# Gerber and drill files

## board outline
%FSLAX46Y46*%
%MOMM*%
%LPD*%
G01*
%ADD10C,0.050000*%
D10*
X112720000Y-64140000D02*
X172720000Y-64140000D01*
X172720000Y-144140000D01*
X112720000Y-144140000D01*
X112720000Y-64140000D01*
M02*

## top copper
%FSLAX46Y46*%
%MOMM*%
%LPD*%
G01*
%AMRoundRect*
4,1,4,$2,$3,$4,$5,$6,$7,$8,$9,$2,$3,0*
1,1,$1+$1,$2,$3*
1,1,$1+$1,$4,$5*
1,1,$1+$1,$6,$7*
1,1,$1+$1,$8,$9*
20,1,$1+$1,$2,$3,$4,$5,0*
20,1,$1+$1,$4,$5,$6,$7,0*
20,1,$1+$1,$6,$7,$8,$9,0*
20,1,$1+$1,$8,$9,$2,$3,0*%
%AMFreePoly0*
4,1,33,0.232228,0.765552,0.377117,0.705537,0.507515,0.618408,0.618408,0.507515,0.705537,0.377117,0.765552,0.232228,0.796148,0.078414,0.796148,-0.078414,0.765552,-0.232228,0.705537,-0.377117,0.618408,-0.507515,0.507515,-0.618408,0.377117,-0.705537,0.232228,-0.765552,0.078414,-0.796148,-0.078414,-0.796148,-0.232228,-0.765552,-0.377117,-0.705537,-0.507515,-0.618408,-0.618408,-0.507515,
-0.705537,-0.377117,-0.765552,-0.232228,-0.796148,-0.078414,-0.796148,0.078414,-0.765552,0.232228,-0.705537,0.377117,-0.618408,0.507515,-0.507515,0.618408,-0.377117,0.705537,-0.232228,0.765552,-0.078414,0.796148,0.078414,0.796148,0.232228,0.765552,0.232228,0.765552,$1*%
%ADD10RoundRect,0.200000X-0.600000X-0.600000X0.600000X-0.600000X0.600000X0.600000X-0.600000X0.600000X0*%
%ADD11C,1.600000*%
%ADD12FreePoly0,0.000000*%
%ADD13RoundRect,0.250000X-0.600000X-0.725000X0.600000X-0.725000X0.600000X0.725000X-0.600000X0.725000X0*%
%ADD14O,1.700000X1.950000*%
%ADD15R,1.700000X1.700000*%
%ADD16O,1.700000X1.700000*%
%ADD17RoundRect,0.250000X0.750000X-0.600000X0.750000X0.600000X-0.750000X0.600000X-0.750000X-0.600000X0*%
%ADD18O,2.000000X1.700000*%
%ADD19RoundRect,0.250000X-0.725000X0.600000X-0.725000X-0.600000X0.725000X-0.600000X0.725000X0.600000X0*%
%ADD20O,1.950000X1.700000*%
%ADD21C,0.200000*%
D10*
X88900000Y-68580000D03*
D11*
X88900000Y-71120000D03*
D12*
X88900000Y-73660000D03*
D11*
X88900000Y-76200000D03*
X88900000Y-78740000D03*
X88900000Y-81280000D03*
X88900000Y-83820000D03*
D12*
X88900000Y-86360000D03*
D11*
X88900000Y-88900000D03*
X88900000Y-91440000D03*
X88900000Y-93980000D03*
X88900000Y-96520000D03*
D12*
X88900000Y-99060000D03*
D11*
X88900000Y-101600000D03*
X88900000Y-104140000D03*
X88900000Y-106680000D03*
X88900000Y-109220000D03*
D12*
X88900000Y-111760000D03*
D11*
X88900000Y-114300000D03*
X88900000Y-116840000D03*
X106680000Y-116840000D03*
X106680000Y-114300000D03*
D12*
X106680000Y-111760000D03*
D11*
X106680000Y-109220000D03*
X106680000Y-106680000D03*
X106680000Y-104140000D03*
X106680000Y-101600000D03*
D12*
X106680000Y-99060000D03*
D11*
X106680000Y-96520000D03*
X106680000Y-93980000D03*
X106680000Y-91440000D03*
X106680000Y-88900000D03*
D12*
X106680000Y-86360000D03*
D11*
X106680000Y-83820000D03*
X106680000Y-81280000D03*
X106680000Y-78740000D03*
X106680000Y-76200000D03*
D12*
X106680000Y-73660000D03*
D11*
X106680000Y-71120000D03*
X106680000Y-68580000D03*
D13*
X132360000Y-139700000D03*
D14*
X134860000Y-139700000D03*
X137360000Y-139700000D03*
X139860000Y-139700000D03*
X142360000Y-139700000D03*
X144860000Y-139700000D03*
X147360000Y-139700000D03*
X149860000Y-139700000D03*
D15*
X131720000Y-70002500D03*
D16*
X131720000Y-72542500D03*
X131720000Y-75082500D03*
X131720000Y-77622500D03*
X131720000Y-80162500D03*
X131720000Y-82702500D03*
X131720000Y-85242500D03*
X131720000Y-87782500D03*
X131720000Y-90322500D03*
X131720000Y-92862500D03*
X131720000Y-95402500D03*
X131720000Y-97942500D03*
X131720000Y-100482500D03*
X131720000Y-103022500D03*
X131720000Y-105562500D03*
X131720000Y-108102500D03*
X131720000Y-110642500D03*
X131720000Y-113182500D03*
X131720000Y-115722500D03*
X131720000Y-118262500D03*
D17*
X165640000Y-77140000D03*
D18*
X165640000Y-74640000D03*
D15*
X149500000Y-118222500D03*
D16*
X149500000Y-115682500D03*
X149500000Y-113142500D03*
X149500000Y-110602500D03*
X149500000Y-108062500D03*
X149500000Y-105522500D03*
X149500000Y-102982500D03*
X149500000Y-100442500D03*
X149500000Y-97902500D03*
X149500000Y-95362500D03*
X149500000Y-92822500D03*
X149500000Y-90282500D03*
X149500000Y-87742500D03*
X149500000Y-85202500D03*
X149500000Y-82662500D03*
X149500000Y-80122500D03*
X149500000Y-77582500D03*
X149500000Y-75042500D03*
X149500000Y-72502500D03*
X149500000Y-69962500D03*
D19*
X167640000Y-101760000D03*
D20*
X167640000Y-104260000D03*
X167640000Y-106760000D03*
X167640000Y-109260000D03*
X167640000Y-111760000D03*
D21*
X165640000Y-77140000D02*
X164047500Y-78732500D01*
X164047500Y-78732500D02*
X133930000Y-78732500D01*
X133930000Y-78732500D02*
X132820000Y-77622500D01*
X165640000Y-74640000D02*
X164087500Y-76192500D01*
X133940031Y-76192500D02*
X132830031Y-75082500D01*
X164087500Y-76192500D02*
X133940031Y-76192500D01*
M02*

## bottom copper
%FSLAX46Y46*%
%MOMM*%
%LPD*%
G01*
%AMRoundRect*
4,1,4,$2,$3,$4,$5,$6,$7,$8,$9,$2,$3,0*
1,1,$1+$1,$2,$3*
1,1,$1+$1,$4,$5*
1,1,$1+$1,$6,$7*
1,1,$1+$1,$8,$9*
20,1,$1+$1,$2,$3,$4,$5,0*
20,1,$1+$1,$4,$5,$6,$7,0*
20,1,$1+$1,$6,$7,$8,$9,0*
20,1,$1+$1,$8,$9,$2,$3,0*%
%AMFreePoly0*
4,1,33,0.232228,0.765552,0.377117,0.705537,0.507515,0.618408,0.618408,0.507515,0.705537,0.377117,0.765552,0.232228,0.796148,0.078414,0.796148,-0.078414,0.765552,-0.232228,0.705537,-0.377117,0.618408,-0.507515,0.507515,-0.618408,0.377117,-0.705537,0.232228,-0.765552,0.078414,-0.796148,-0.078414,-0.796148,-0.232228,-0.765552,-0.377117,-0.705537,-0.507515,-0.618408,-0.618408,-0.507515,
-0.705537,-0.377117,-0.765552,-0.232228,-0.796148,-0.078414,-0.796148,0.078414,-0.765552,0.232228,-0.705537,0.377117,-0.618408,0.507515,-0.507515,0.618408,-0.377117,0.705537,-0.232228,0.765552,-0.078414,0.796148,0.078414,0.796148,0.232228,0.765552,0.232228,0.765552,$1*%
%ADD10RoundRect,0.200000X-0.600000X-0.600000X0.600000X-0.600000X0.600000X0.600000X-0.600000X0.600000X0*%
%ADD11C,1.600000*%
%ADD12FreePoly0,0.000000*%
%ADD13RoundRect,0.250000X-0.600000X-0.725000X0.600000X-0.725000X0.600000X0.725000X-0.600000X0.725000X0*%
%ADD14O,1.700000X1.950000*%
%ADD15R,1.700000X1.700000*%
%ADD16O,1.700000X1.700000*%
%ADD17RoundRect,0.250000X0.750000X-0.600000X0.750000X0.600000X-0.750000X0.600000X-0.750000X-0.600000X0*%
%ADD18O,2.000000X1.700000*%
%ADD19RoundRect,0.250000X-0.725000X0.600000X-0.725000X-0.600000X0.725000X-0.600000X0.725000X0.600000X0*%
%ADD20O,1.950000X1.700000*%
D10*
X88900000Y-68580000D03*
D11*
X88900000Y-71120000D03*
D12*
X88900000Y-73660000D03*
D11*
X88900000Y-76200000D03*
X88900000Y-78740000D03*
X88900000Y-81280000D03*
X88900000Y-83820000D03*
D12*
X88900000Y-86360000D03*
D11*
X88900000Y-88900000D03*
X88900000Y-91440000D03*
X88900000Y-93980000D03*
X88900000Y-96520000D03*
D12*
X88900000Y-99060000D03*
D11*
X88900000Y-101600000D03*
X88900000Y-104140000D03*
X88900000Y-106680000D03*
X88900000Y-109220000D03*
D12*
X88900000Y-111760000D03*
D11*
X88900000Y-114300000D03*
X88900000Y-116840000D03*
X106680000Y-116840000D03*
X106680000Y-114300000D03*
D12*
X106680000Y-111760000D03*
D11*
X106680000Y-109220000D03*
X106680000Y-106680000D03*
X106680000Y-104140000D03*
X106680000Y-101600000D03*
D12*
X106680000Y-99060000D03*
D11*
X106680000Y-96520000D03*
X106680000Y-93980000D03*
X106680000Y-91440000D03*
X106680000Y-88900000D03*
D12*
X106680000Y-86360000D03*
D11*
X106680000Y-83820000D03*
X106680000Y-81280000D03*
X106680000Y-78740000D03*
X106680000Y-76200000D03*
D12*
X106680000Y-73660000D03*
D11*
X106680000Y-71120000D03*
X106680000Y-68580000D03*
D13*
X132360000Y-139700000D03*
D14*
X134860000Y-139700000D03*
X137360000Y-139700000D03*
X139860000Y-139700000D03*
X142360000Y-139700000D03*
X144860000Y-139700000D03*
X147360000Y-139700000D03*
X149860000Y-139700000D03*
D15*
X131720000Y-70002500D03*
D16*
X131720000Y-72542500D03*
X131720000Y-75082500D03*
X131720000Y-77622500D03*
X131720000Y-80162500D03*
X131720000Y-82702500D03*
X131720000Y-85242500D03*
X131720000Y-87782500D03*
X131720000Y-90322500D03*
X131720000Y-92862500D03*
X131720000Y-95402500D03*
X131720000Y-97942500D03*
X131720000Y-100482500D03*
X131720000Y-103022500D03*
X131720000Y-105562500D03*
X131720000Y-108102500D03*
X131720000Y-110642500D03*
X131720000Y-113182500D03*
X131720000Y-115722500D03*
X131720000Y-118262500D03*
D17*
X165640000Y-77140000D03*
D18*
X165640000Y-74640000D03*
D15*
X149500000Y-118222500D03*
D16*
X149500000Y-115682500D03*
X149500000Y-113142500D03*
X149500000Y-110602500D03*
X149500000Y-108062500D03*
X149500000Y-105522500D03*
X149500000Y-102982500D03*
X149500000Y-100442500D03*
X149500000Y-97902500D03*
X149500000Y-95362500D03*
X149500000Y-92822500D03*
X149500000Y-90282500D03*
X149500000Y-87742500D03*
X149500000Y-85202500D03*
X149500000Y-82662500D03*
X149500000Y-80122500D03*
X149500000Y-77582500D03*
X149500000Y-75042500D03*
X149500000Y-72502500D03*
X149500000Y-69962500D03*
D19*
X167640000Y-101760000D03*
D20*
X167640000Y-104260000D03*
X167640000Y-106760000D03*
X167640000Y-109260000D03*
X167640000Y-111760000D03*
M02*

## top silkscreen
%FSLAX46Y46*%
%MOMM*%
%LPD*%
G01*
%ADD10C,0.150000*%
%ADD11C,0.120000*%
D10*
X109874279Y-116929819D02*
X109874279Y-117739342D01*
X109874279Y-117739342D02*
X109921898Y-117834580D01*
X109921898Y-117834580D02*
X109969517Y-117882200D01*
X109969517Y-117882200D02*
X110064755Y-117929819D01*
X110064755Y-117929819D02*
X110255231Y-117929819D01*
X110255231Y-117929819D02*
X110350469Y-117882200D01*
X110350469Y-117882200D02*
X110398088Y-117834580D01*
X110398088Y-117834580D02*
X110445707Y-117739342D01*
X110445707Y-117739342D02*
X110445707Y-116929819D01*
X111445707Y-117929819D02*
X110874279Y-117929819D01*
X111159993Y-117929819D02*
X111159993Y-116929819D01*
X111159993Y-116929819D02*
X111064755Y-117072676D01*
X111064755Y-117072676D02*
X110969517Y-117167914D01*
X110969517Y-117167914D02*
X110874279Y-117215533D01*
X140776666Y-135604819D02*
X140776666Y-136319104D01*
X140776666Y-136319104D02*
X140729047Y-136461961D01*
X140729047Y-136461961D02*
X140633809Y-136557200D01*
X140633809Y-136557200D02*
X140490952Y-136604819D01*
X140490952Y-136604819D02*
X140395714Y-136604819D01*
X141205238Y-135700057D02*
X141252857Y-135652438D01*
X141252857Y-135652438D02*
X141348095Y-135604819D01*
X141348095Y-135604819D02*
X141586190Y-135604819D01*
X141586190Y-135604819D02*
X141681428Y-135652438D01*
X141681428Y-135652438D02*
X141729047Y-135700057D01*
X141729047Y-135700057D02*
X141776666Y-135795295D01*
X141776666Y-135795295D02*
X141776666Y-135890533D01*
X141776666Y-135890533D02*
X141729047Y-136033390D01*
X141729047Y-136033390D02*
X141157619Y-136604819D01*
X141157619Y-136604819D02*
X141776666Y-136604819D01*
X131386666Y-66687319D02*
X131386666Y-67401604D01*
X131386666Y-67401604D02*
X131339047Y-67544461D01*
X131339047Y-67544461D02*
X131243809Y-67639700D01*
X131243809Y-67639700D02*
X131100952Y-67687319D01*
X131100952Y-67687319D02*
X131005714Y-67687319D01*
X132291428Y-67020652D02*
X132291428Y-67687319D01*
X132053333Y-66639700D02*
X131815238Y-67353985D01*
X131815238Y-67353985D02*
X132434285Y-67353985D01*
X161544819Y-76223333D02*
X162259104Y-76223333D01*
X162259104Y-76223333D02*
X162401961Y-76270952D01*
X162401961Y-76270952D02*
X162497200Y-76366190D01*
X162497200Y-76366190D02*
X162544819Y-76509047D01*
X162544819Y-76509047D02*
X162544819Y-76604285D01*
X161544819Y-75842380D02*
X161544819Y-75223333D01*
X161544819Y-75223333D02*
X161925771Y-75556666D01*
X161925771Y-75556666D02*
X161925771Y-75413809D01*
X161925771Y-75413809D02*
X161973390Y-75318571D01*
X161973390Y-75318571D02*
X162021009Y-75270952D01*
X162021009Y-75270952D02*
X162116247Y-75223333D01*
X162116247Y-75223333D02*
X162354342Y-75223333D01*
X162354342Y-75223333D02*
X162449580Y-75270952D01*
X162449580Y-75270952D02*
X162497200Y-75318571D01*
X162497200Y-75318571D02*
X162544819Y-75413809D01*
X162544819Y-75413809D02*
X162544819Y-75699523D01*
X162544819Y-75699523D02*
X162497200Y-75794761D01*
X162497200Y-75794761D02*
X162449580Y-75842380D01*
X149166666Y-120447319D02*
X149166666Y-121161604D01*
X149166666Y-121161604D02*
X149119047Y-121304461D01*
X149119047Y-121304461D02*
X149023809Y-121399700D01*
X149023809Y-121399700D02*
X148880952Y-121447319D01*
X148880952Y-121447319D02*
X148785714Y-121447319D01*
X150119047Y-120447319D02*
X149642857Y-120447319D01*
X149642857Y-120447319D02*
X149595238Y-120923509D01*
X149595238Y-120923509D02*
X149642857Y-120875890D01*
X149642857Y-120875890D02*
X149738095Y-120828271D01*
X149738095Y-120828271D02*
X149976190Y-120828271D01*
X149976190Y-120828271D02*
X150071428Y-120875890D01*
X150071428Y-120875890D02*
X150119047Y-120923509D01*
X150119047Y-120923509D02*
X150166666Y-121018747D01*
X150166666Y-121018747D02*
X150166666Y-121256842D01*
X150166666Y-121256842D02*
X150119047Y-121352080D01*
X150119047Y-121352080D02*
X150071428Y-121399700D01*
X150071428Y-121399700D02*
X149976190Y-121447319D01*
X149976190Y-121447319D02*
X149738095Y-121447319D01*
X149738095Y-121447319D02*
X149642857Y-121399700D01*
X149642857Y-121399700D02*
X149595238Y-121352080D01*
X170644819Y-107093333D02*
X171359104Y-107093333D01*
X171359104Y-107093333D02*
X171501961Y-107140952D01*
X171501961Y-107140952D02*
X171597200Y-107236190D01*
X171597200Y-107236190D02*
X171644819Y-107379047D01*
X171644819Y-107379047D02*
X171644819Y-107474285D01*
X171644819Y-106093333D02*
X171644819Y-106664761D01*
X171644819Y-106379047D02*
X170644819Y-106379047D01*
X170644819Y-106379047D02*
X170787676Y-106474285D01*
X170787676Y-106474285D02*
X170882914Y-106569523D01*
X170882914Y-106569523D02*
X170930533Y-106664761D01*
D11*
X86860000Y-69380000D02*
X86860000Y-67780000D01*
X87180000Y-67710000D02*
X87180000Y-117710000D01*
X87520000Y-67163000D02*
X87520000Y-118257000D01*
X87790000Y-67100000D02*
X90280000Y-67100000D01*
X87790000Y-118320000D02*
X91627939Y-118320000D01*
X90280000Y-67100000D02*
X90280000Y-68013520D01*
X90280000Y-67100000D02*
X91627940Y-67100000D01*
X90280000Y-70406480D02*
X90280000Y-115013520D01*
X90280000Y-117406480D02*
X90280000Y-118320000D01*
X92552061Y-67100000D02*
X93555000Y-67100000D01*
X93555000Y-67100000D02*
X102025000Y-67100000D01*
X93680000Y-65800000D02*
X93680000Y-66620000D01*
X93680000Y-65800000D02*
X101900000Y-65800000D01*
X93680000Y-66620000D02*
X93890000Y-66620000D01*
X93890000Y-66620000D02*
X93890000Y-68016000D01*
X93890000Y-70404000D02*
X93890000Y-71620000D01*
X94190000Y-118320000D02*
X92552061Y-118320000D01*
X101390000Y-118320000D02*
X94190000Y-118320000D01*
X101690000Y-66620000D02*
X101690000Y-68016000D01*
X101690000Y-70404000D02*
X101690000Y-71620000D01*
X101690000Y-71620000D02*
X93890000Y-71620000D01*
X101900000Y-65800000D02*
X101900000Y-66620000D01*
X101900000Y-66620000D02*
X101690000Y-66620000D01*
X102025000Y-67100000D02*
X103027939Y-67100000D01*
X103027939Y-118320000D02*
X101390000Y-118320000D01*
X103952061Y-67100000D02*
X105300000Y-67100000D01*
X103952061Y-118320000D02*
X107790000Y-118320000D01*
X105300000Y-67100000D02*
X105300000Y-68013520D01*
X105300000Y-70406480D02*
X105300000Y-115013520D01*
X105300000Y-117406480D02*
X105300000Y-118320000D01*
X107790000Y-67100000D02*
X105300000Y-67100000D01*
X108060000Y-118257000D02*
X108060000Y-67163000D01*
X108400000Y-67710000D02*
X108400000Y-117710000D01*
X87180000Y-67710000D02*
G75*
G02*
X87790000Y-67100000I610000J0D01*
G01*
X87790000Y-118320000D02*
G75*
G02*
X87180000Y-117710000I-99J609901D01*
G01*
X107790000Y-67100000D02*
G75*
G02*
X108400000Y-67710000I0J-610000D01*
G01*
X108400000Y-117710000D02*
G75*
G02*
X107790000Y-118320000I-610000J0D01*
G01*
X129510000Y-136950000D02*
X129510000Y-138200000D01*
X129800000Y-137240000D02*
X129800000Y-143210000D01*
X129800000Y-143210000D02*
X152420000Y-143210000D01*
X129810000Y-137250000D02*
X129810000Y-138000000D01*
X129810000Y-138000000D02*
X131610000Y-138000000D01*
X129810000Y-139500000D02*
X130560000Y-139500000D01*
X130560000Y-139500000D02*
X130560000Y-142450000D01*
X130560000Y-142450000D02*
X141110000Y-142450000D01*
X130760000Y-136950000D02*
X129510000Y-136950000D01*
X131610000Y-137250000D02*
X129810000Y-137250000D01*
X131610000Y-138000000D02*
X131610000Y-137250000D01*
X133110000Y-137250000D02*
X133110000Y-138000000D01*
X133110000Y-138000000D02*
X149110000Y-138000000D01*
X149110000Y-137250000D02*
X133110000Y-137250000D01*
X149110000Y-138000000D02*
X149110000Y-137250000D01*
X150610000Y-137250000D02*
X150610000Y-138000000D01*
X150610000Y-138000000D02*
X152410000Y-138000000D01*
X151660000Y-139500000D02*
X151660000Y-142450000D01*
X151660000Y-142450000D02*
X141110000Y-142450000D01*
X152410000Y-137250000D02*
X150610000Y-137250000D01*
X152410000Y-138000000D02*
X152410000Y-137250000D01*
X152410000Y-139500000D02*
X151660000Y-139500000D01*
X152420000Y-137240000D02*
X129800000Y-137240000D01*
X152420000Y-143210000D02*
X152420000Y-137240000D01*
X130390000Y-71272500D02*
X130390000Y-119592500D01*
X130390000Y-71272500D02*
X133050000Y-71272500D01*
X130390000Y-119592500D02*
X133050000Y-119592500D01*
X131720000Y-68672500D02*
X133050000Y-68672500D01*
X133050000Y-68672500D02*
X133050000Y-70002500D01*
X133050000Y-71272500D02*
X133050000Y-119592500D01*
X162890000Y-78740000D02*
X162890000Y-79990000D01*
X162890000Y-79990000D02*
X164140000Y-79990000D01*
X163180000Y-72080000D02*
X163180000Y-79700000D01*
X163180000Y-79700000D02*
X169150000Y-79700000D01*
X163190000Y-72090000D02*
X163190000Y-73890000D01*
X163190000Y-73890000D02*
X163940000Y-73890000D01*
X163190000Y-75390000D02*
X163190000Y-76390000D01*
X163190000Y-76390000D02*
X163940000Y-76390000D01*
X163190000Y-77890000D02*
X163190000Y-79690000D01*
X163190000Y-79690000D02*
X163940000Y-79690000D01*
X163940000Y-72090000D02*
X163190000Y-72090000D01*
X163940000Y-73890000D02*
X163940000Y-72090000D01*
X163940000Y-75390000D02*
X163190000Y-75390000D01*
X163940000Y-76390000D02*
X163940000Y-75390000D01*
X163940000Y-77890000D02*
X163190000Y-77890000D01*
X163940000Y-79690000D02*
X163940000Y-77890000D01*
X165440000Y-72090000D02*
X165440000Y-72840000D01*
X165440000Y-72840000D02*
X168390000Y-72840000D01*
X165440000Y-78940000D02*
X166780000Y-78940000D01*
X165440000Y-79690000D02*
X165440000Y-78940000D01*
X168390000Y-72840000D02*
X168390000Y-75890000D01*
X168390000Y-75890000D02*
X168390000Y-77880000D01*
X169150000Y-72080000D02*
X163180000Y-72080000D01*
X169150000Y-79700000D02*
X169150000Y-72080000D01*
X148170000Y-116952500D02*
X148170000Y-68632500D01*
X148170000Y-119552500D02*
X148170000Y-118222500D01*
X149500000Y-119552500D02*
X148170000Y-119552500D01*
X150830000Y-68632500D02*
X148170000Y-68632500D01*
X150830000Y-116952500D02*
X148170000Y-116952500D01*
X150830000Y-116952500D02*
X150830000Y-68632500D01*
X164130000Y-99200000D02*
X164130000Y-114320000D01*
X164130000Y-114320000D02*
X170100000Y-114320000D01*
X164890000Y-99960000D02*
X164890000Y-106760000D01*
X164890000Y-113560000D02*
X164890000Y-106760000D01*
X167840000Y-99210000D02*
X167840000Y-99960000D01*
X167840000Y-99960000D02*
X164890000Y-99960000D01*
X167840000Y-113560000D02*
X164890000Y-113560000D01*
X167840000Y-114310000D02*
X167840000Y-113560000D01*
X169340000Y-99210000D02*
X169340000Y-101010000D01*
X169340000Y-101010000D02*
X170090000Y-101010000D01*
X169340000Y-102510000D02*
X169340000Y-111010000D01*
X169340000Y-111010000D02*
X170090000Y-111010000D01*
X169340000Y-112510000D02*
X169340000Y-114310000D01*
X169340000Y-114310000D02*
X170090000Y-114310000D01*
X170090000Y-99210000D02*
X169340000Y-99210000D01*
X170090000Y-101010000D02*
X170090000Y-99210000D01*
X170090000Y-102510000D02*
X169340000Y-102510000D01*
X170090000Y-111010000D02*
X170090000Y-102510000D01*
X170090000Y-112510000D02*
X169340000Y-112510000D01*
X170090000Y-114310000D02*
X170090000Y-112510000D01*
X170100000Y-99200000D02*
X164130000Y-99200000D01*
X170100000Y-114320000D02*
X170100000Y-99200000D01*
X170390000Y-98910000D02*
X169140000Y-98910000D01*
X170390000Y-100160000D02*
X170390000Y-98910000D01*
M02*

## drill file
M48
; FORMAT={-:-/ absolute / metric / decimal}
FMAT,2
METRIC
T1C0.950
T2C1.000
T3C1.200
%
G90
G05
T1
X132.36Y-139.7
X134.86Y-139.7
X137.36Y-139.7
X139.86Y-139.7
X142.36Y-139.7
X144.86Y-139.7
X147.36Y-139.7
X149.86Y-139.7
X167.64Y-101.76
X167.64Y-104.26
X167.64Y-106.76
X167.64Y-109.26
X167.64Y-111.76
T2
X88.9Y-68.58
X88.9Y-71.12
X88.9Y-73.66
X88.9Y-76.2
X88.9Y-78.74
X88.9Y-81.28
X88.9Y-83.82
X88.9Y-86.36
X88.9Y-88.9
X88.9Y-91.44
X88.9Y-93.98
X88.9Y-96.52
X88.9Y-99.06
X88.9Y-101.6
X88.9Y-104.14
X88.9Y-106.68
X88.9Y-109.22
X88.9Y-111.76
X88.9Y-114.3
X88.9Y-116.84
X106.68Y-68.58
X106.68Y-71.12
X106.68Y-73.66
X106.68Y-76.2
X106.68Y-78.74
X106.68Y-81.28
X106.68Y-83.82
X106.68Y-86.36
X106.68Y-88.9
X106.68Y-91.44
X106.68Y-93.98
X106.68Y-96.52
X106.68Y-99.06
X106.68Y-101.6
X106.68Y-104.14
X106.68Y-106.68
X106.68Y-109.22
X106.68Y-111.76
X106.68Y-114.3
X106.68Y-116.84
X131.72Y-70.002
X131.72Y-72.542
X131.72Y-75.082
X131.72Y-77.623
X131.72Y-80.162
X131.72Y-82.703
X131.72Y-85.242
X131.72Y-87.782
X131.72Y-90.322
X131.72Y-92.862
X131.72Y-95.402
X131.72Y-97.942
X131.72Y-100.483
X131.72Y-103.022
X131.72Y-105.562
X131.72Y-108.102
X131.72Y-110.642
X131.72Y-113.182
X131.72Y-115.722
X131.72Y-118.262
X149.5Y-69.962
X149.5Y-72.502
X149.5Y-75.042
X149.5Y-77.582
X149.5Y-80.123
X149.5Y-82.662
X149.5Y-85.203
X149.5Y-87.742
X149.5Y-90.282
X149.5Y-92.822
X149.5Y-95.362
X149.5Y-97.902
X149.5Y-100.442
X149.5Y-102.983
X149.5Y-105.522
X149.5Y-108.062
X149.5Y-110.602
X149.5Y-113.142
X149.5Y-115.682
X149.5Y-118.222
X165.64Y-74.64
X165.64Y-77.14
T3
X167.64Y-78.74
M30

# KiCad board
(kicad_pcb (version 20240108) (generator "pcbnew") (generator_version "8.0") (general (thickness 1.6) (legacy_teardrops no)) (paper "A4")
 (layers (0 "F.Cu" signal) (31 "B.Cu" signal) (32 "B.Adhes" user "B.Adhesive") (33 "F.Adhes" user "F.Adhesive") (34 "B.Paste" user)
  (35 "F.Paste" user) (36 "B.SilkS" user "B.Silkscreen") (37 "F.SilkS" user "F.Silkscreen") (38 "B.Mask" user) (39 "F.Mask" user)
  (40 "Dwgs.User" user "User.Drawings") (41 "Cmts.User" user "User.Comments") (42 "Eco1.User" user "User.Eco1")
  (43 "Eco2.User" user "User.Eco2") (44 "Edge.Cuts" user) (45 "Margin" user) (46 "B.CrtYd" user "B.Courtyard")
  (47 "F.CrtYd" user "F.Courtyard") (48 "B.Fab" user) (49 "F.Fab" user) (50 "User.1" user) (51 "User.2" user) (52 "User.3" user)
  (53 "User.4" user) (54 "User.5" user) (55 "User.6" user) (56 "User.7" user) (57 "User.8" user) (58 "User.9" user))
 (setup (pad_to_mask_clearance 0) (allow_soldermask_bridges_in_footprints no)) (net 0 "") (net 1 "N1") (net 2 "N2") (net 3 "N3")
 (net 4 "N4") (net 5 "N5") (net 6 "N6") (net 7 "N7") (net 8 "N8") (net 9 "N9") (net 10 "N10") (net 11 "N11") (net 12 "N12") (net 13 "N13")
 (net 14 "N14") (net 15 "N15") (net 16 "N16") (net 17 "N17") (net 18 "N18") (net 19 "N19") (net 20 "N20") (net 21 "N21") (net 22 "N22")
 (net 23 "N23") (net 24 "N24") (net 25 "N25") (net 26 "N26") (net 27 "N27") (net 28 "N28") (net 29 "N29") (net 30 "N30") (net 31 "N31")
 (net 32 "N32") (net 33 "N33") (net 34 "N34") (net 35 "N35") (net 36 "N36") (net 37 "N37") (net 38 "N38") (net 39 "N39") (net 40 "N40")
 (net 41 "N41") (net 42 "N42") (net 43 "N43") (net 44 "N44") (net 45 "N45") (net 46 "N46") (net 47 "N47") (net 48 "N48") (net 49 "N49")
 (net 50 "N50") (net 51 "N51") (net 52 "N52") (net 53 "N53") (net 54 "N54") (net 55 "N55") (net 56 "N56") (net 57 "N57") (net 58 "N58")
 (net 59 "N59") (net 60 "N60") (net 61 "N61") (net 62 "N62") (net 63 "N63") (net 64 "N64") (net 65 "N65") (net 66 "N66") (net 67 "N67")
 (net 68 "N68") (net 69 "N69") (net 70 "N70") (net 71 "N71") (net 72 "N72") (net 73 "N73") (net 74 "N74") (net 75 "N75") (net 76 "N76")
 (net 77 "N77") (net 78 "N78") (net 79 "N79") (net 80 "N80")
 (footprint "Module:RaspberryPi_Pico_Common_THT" (layer "F.Cu") (at 88.9 68.58)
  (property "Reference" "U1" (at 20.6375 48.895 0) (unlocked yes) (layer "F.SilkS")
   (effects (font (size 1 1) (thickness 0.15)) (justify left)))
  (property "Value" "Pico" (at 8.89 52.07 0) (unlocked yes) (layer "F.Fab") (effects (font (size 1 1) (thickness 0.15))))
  (fp_line (start -2.04 0.8) (end -2.04 -0.8) (stroke (width 0.12) (type solid)) (layer "F.SilkS"))
  (fp_line (start -1.72 -0.87) (end -1.72 49.13) (stroke (width 0.12) (type solid)) (layer "F.SilkS"))
  (fp_line (start -1.38 -1.417) (end -1.38 49.677) (stroke (width 0.12) (type solid)) (layer "F.SilkS"))
  (fp_line (start -1.11 -1.48) (end 1.38 -1.48) (stroke (width 0.12) (type solid)) (layer "F.SilkS"))
  (fp_line (start -1.11 49.74) (end 2.727939 49.74) (stroke (width 0.12) (type solid)) (layer "F.SilkS"))
  (fp_line (start 1.38 -1.48) (end 1.38 -0.56648) (stroke (width 0.12) (type solid)) (layer "F.SilkS"))
  (fp_line (start 1.38 -1.48) (end 2.72794 -1.48) (stroke (width 0.12) (type solid)) (layer "F.SilkS"))
  (fp_line (start 1.38 1.82648) (end 1.38 46.43352) (stroke (width 0.12) (type solid)) (layer "F.SilkS"))
  (fp_line (start 1.38 48.82648) (end 1.38 49.74) (stroke (width 0.12) (type solid)) (layer "F.SilkS"))
  (fp_line (start 3.652061 -1.48) (end 4.655 -1.48) (stroke (width 0.12) (type solid)) (layer "F.SilkS"))
  (fp_line (start 4.655 -1.48) (end 13.125 -1.48) (stroke (width 0.12) (type solid)) (layer "F.SilkS"))
  (fp_line (start 4.78 -2.78) (end 4.78 -1.96) (stroke (width 0.12) (type solid)) (layer "F.SilkS"))
  (fp_line (start 4.78 -2.78) (end 13 -2.78) (stroke (width 0.12) (type solid)) (layer "F.SilkS"))
  (fp_line (start 4.78 -1.96) (end 4.99 -1.96) (stroke (width 0.12) (type solid)) (layer "F.SilkS"))
  (fp_line (start 4.99 -1.96) (end 4.99 -0.564) (stroke (width 0.12) (type solid)) (layer "F.SilkS"))
  (fp_line (start 4.99 1.824) (end 4.99 3.04) (stroke (width 0.12) (type solid)) (layer "F.SilkS"))
  (fp_line (start 5.29 49.74) (end 3.652061 49.74) (stroke (width 0.12) (type solid)) (layer "F.SilkS"))
  (fp_line (start 12.49 49.74) (end 5.29 49.74) (stroke (width 0.12) (type solid)) (layer "F.SilkS"))
  (fp_line (start 12.79 -1.96) (end 12.79 -0.564) (stroke (width 0.12) (type solid)) (layer "F.SilkS"))
  (fp_line (start 12.79 1.824) (end 12.79 3.04) (stroke (width 0.12) (type solid)) (layer "F.SilkS"))
  (fp_line (start 12.79 3.04) (end 4.99 3.04) (stroke (width 0.12) (type solid)) (layer "F.SilkS"))
  (fp_line (start 13 -2.78) (end 13 -1.96) (stroke (width 0.12) (type solid)) (layer "F.SilkS"))
  (fp_line (start 13 -1.96) (end 12.79 -1.96) (stroke (width 0.12) (type solid)) (layer "F.SilkS"))
  (fp_line (start 13.125 -1.48) (end 14.127939 -1.48) (stroke (width 0.12) (type solid)) (layer "F.SilkS"))
  (fp_line (start 14.127939 49.74) (end 12.49 49.74) (stroke (width 0.12) (type solid)) (layer "F.SilkS"))
  (fp_line (start 15.052061 -1.48) (end 16.4 -1.48) (stroke (width 0.12) (type solid)) (layer "F.SilkS"))
  (fp_line (start 15.052061 49.74) (end 18.89 49.74) (stroke (width 0.12) (type solid)) (layer "F.SilkS"))
  (fp_line (start 16.4 -1.48) (end 16.4 -0.56648) (stroke (width 0.12) (type solid)) (layer "F.SilkS"))
  (fp_line (start 16.4 1.82648) (end 16.4 46.43352) (stroke (width 0.12) (type solid)) (layer "F.SilkS"))
  (fp_line (start 16.4 48.82648) (end 16.4 49.74) (stroke (width 0.12) (type solid)) (layer "F.SilkS"))
  (fp_line (start 18.89 -1.48) (end 16.4 -1.48) (stroke (width 0.12) (type solid)) (layer "F.SilkS"))
  (fp_line (start 19.16 49.677) (end 19.16 -1.417) (stroke (width 0.12) (type solid)) (layer "F.SilkS"))
  (fp_line (start 19.5 -0.87) (end 19.5 49.13) (stroke (width 0.12) (type solid)) (layer "F.SilkS"))
  (fp_arc (start -1.72 -0.87) (mid -1.541335 -1.301335) (end -1.11 -1.48) (stroke (width 0.12) (type solid)) (layer "F.SilkS"))
  (fp_arc (start -1.11 49.74) (mid -1.541364 49.561364) (end -1.72 49.13) (stroke (width 0.12) (type solid)) (layer "F.SilkS"))
  (fp_arc (start 18.89 -1.48) (mid 19.321335 -1.301335) (end 19.5 -0.87) (stroke (width 0.12) (type solid)) (layer "F.SilkS"))
  (fp_arc (start 19.5 49.13) (mid 19.321335 49.561335) (end 18.89 49.74) (stroke (width 0.12) (type solid)) (layer "F.SilkS"))
  (pad "1" thru_hole roundrect (at 0 0) (size 1.6 1.6) (drill 1) (layers "*.Cu" "*.Mask") (remove_unused_layers no) (roundrect_rratio 0.125)
   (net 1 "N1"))
  (pad "2" thru_hole circle (at 0 2.54) (size 1.6 1.6) (drill 1) (layers "*.Cu" "*.Mask") (remove_unused_layers no) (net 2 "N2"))
  (pad "3" thru_hole custom (at 0 5.08) (size 1.6 1.6) (drill 1) (layers "*.Cu" "*.Mask") (remove_unused_layers no) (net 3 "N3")
   (options (clearance outline) (anchor circle)) (primitives))
  (pad "4" thru_hole circle (at 0 7.62) (size 1.6 1.6) (drill 1) (layers "*.Cu" "*.Mask") (remove_unused_layers no) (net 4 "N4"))
  (pad "5" thru_hole circle (at 0 10.16) (size 1.6 1.6) (drill 1) (layers "*.Cu" "*.Mask") (remove_unused_layers no) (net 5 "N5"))
  (pad "6" thru_hole circle (at 0 12.7) (size 1.6 1.6) (drill 1) (layers "*.Cu" "*.Mask") (remove_unused_layers no) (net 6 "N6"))
  (pad "7" thru_hole circle (at 0 15.24) (size 1.6 1.6) (drill 1) (layers "*.Cu" "*.Mask") (remove_unused_layers no) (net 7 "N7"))
  (pad "8" thru_hole custom (at 0 17.78) (size 1.6 1.6) (drill 1) (layers "*.Cu" "*.Mask") (remove_unused_layers no) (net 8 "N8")
   (options (clearance outline) (anchor circle)) (primitives))
  (pad "9" thru_hole circle (at 0 20.32) (size 1.6 1.6) (drill 1) (layers "*.Cu" "*.Mask") (remove_unused_layers no) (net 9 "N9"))
  (pad "10" thru_hole circle (at 0 22.86) (size 1.6 1.6) (drill 1) (layers "*.Cu" "*.Mask") (remove_unused_layers no) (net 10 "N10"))
  (pad "11" thru_hole circle (at 0 25.4) (size 1.6 1.6) (drill 1) (layers "*.Cu" "*.Mask") (remove_unused_layers no) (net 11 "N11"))
  (pad "12" thru_hole circle (at 0 27.94) (size 1.6 1.6) (drill 1) (layers "*.Cu" "*.Mask") (remove_unused_layers no) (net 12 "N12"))
  (pad "13" thru_hole custom (at 0 30.48) (size 1.6 1.6) (drill 1) (layers "*.Cu" "*.Mask") (remove_unused_layers no) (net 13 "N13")
   (options (clearance outline) (anchor circle)) (primitives))
  (pad "14" thru_hole circle (at 0 33.02) (size 1.6 1.6) (drill 1) (layers "*.Cu" "*.Mask") (remove_unused_layers no) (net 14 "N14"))
  (pad "15" thru_hole circle (at 0 35.56) (size 1.6 1.6) (drill 1) (layers "*.Cu" "*.Mask") (remove_unused_layers no) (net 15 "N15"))
  (pad "16" thru_hole circle (at 0 38.1) (size 1.6 1.6) (drill 1) (layers "*.Cu" "*.Mask") (remove_unused_layers no) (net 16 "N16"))
  (pad "17" thru_hole circle (at 0 40.64) (size 1.6 1.6) (drill 1) (layers "*.Cu" "*.Mask") (remove_unused_layers no) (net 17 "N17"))
  (pad "18" thru_hole custom (at 0 43.18) (size 1.6 1.6) (drill 1) (layers "*.Cu" "*.Mask") (remove_unused_layers no) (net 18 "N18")
   (options (clearance outline) (anchor circle)) (primitives))
  (pad "19" thru_hole circle (at 0 45.72) (size 1.6 1.6) (drill 1) (layers "*.Cu" "*.Mask") (remove_unused_layers no) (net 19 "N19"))
  (pad "20" thru_hole circle (at 0 48.26) (size 1.6 1.6) (drill 1) (layers "*.Cu" "*.Mask") (remove_unused_layers no) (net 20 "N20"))
  (pad "21" thru_hole circle (at 17.78 48.26) (size 1.6 1.6) (drill 1) (layers "*.Cu" "*.Mask") (remove_unused_layers no) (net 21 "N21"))
  (pad "22" thru_hole circle (at 17.78 45.72) (size 1.6 1.6) (drill 1) (layers "*.Cu" "*.Mask") (remove_unused_layers no) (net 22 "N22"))
  (pad "23" thru_hole custom (at 17.78 43.18) (size 1.6 1.6) (drill 1) (layers "*.Cu" "*.Mask") (remove_unused_layers no) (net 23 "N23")
   (options (clearance outline) (anchor circle)) (primitives))
  (pad "24" thru_hole circle (at 17.78 40.64) (size 1.6 1.6) (drill 1) (layers "*.Cu" "*.Mask") (remove_unused_layers no) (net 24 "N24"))
  (pad "25" thru_hole circle (at 17.78 38.1) (size 1.6 1.6) (drill 1) (layers "*.Cu" "*.Mask") (remove_unused_layers no) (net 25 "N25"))
  (pad "26" thru_hole circle (at 17.78 35.56) (size 1.6 1.6) (drill 1) (layers "*.Cu" "*.Mask") (remove_unused_layers no) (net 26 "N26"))
  (pad "27" thru_hole circle (at 17.78 33.02) (size 1.6 1.6) (drill 1) (layers "*.Cu" "*.Mask") (remove_unused_layers no) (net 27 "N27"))
  (pad "28" thru_hole custom (at 17.78 30.48) (size 1.6 1.6) (drill 1) (layers "*.Cu" "*.Mask") (remove_unused_layers no) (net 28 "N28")
   (options (clearance outline) (anchor circle)) (primitives))
  (pad "29" thru_hole circle (at 17.78 27.94) (size 1.6 1.6) (drill 1) (layers "*.Cu" "*.Mask") (remove_unused_layers no) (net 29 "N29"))
  (pad "30" thru_hole circle (at 17.78 25.4) (size 1.6 1.6) (drill 1) (layers "*.Cu" "*.Mask") (remove_unused_layers no) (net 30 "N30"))
  (pad "31" thru_hole circle (at 17.78 22.86) (size 1.6 1.6) (drill 1) (layers "*.Cu" "*.Mask") (remove_unused_layers no) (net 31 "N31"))
  (pad "32" thru_hole circle (at 17.78 20.32) (size 1.6 1.6) (drill 1) (layers "*.Cu" "*.Mask") (remove_unused_layers no) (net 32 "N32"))
  (pad "33" thru_hole custom (at 17.78 17.78) (size 1.6 1.6) (drill 1) (layers "*.Cu" "*.Mask") (remove_unused_layers no) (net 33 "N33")
   (options (clearance outline) (anchor circle)) (primitives))
  (pad "34" thru_hole circle (at 17.78 15.24) (size 1.6 1.6) (drill 1) (layers "*.Cu" "*.Mask") (remove_unused_layers no) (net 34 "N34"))
  (pad "35" thru_hole circle (at 17.78 12.7) (size 1.6 1.6) (drill 1) (layers "*.Cu" "*.Mask") (remove_unused_layers no) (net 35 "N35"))
  (pad "36" thru_hole circle (at 17.78 10.16) (size 1.6 1.6) (drill 1) (layers "*.Cu" "*.Mask") (remove_unused_layers no) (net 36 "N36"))
  (pad "37" thru_hole circle (at 17.78 7.62) (size 1.6 1.6) (drill 1) (layers "*.Cu" "*.Mask") (remove_unused_layers no) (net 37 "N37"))
  (pad "38" thru_hole custom (at 17.78 5.08) (size 1.6 1.6) (drill 1) (layers "*.Cu" "*.Mask") (remove_unused_layers no) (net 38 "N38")
   (options (clearance outline) (anchor circle)) (primitives))
  (pad "39" thru_hole circle (at 17.78 2.54) (size 1.6 1.6) (drill 1) (layers "*.Cu" "*.Mask") (remove_unused_layers no) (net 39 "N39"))
  (pad "40" thru_hole circle (at 17.78 0) (size 1.6 1.6) (drill 1) (layers "*.Cu" "*.Mask") (remove_unused_layers no) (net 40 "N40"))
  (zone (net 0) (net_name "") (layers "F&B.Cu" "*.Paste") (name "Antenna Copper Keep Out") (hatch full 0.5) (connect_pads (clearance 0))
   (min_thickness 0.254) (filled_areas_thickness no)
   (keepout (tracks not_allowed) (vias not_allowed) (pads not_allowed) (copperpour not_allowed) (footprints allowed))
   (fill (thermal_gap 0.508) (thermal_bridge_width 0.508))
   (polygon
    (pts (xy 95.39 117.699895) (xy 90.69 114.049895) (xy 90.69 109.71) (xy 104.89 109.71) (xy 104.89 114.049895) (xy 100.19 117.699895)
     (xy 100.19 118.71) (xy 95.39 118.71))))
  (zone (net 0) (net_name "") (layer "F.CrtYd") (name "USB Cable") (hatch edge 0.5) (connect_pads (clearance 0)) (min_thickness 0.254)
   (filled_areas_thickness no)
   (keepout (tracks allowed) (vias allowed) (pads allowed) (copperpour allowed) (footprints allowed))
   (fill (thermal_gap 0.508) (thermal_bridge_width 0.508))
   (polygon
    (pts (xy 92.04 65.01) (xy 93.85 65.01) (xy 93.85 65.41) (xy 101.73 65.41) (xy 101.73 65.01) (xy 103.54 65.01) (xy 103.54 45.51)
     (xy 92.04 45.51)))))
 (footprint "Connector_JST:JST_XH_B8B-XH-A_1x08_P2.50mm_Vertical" (layer "F.Cu") (at 132.36 139.7)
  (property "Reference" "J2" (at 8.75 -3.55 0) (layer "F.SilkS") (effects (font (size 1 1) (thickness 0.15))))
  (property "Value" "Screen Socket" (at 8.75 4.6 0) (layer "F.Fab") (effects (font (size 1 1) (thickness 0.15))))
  (fp_line (start -2.85 -2.75) (end -2.85 -1.5) (stroke (width 0.12) (type solid)) (layer "F.SilkS"))
  (fp_line (start -2.56 -2.46) (end -2.56 3.51) (stroke (width 0.12) (type solid)) (layer "F.SilkS"))
  (fp_line (start -2.56 3.51) (end 20.06 3.51) (stroke (width 0.12) (type solid)) (layer "F.SilkS"))
  (fp_line (start -2.55 -2.45) (end -2.55 -1.7) (stroke (width 0.12) (type solid)) (layer "F.SilkS"))
  (fp_line (start -2.55 -1.7) (end -0.75 -1.7) (stroke (width 0.12) (type solid)) (layer "F.SilkS"))
  (fp_line (start -2.55 -0.2) (end -1.8 -0.2) (stroke (width 0.12) (type solid)) (layer "F.SilkS"))
  (fp_line (start -1.8 -0.2) (end -1.8 2.75) (stroke (width 0.12) (type solid)) (layer "F.SilkS"))
  (fp_line (start -1.8 2.75) (end 8.75 2.75) (stroke (width 0.12) (type solid)) (layer "F.SilkS"))
  (fp_line (start -1.6 -2.75) (end -2.85 -2.75) (stroke (width 0.12) (type solid)) (layer "F.SilkS"))
  (fp_line (start -0.75 -2.45) (end -2.55 -2.45) (stroke (width 0.12) (type solid)) (layer "F.SilkS"))
  (fp_line (start -0.75 -1.7) (end -0.75 -2.45) (stroke (width 0.12) (type solid)) (layer "F.SilkS"))
  (fp_line (start 0.75 -2.45) (end 0.75 -1.7) (stroke (width 0.12) (type solid)) (layer "F.SilkS"))
  (fp_line (start 0.75 -1.7) (end 16.75 -1.7) (stroke (width 0.12) (type solid)) (layer "F.SilkS"))
  (fp_line (start 16.75 -2.45) (end 0.75 -2.45) (stroke (width 0.12) (type solid)) (layer "F.SilkS"))
  (fp_line (start 16.75 -1.7) (end 16.75 -2.45) (stroke (width 0.12) (type solid)) (layer "F.SilkS"))
  (fp_line (start 18.25 -2.45) (end 18.25 -1.7) (stroke (width 0.12) (type solid)) (layer "F.SilkS"))
  (fp_line (start 18.25 -1.7) (end 20.05 -1.7) (stroke (width 0.12) (type solid)) (layer "F.SilkS"))
  (fp_line (start 19.3 -0.2) (end 19.3 2.75) (stroke (width 0.12) (type solid)) (layer "F.SilkS"))
  (fp_line (start 19.3 2.75) (end 8.75 2.75) (stroke (width 0.12) (type solid)) (layer "F.SilkS"))
  (fp_line (start 20.05 -2.45) (end 18.25 -2.45) (stroke (width 0.12) (type solid)) (layer "F.SilkS"))
  (fp_line (start 20.05 -1.7) (end 20.05 -2.45) (stroke (width 0.12) (type solid)) (layer "F.SilkS"))
  (fp_line (start 20.05 -0.2) (end 19.3 -0.2) (stroke (width 0.12) (type solid)) (layer "F.SilkS"))
  (fp_line (start 20.06 -2.46) (end -2.56 -2.46) (stroke (width 0.12) (type solid)) (layer "F.SilkS"))
  (fp_line (start 20.06 3.51) (end 20.06 -2.46) (stroke (width 0.12) (type solid)) (layer "F.SilkS"))
  (pad "1" thru_hole roundrect (at 0 0) (size 1.7 1.95) (drill 0.95) (layers "*.Cu" "*.Mask") (remove_unused_layers no)
   (roundrect_rratio 0.147059) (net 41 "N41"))
  (pad "2" thru_hole oval (at 2.5 0) (size 1.7 1.95) (drill 0.95) (layers "*.Cu" "*.Mask") (remove_unused_layers no) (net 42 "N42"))
  (pad "3" thru_hole oval (at 5 0) (size 1.7 1.95) (drill 0.95) (layers "*.Cu" "*.Mask") (remove_unused_layers no) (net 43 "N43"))
  (pad "4" thru_hole oval (at 7.5 0) (size 1.7 1.95) (drill 0.95) (layers "*.Cu" "*.Mask") (remove_unused_layers no) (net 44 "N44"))
  (pad "5" thru_hole oval (at 10 0) (size 1.7 1.95) (drill 0.95) (layers "*.Cu" "*.Mask") (remove_unused_layers no) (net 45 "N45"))
  (pad "6" thru_hole oval (at 12.5 0) (size 1.7 1.95) (drill 0.95) (layers "*.Cu" "*.Mask") (remove_unused_layers no) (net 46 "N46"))
  (pad "7" thru_hole oval (at 15 0) (size 1.7 1.95) (drill 0.95) (layers "*.Cu" "*.Mask") (remove_unused_layers no) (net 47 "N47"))
  (pad "8" thru_hole oval (at 17.5 0) (size 1.7 1.95) (drill 0.95) (layers "*.Cu" "*.Mask") (remove_unused_layers no) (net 41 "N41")))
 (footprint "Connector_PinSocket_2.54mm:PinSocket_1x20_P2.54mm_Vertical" (layer "F.Cu") (at 131.72 70.0025)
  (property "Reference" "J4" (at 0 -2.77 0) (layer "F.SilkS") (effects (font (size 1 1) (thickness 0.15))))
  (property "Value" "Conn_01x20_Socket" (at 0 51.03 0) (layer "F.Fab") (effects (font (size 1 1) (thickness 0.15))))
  (fp_line (start -1.33 1.27) (end -1.33 49.59) (stroke (width 0.12) (type solid)) (layer "F.SilkS"))
  (fp_line (start -1.33 1.27) (end 1.33 1.27) (stroke (width 0.12) (type solid)) (layer "F.SilkS"))
  (fp_line (start -1.33 49.59) (end 1.33 49.59) (stroke (width 0.12) (type solid)) (layer "F.SilkS"))
  (fp_line (start 0 -1.33) (end 1.33 -1.33) (stroke (width 0.12) (type solid)) (layer "F.SilkS"))
  (fp_line (start 1.33 -1.33) (end 1.33 0) (stroke (width 0.12) (type solid)) (layer "F.SilkS"))
  (fp_line (start 1.33 1.27) (end 1.33 49.59) (stroke (width 0.12) (type solid)) (layer "F.SilkS"))
  (pad "1" thru_hole rect (at 0 0) (size 1.7 1.7) (drill 1) (layers "*.Cu" "*.Mask") (remove_unused_layers no) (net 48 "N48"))
  (pad "2" thru_hole oval (at 0 2.54) (size 1.7 1.7) (drill 1) (layers "*.Cu" "*.Mask") (remove_unused_layers no) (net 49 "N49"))
  (pad "3" thru_hole oval (at 0 5.08) (size 1.7 1.7) (drill 1) (layers "*.Cu" "*.Mask") (remove_unused_layers no) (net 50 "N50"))
  (pad "4" thru_hole oval (at 0 7.62) (size 1.7 1.7) (drill 1) (layers "*.Cu" "*.Mask") (remove_unused_layers no) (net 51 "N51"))
  (pad "5" thru_hole oval (at 0 10.16) (size 1.7 1.7) (drill 1) (layers "*.Cu" "*.Mask") (remove_unused_layers no) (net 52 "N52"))
  (pad "6" thru_hole oval (at 0 12.7) (size 1.7 1.7) (drill 1) (layers "*.Cu" "*.Mask") (remove_unused_layers no) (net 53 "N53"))
  (pad "7" thru_hole oval (at 0 15.24) (size 1.7 1.7) (drill 1) (layers "*.Cu" "*.Mask") (remove_unused_layers no) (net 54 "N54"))
  (pad "8" thru_hole oval (at 0 17.78) (size 1.7 1.7) (drill 1) (layers "*.Cu" "*.Mask") (remove_unused_layers no) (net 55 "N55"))
  (pad "9" thru_hole oval (at 0 20.32) (size 1.7 1.7) (drill 1) (layers "*.Cu" "*.Mask") (remove_unused_layers no) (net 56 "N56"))
  (pad "10" thru_hole oval (at 0 22.86) (size 1.7 1.7) (drill 1) (layers "*.Cu" "*.Mask") (remove_unused_layers no) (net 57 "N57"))
  (pad "11" thru_hole oval (at 0 25.4) (size 1.7 1.7) (drill 1) (layers "*.Cu" "*.Mask") (remove_unused_layers no) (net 43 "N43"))
  (pad "12" thru_hole oval (at 0 27.94) (size 1.7 1.7) (drill 1) (layers "*.Cu" "*.Mask") (remove_unused_layers no) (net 44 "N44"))
  (pad "13" thru_hole oval (at 0 30.48) (size 1.7 1.7) (drill 1) (layers "*.Cu" "*.Mask") (remove_unused_layers no) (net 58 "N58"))
  (pad "14" thru_hole oval (at 0 33.02) (size 1.7 1.7) (drill 1) (layers "*.Cu" "*.Mask") (remove_unused_layers no) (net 45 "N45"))
  (pad "15" thru_hole oval (at 0 35.56) (size 1.7 1.7) (drill 1) (layers "*.Cu" "*.Mask") (remove_unused_layers no) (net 46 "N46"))
  (pad "16" thru_hole oval (at 0 38.1) (size 1.7 1.7) (drill 1) (layers "*.Cu" "*.Mask") (remove_unused_layers no) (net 42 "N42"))
  (pad "17" thru_hole oval (at 0 40.64) (size 1.7 1.7) (drill 1) (layers "*.Cu" "*.Mask") (remove_unused_layers no) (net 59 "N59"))
  (pad "18" thru_hole oval (at 0 43.18) (size 1.7 1.7) (drill 1) (layers "*.Cu" "*.Mask") (remove_unused_layers no) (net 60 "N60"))
  (pad "19" thru_hole oval (at 0 45.72) (size 1.7 1.7) (drill 1) (layers "*.Cu" "*.Mask") (remove_unused_layers no) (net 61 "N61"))
  (pad "20" thru_hole oval (at 0 48.26) (size 1.7 1.7) (drill 1) (layers "*.Cu" "*.Mask") (remove_unused_layers no) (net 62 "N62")))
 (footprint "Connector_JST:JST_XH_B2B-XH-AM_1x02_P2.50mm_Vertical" (layer "F.Cu") (at 165.64 77.14 90)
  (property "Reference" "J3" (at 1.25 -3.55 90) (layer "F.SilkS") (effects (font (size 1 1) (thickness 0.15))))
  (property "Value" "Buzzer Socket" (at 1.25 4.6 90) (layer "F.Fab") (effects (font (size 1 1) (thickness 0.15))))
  (fp_line (start -1.6 -2.75) (end -2.85 -2.75) (stroke (width 0.12) (type solid)) (layer "F.SilkS"))
  (fp_line (start -2.85 -2.75) (end -2.85 -1.5) (stroke (width 0.12) (type solid)) (layer "F.SilkS"))
  (fp_line (start 5.06 -2.46) (end -2.56 -2.46) (stroke (width 0.12) (type solid)) (layer "F.SilkS"))
  (fp_line (start -2.56 -2.46) (end -2.56 3.51) (stroke (width 0.12) (type solid)) (layer "F.SilkS"))
  (fp_line (start 5.05 -2.45) (end 3.25 -2.45) (stroke (width 0.12) (type solid)) (layer "F.SilkS"))
  (fp_line (start 3.25 -2.45) (end 3.25 -1.7) (stroke (width 0.12) (type solid)) (layer "F.SilkS"))
  (fp_line (start 1.75 -2.45) (end 0.75 -2.45) (stroke (width 0.12) (type solid)) (layer "F.SilkS"))
  (fp_line (start 0.75 -2.45) (end 0.75 -1.7) (stroke (width 0.12) (type solid)) (layer "F.SilkS"))
  (fp_line (start -0.75 -2.45) (end -2.55 -2.45) (stroke (width 0.12) (type solid)) (layer "F.SilkS"))
  (fp_line (start -2.55 -2.45) (end -2.55 -1.7) (stroke (width 0.12) (type solid)) (layer "F.SilkS"))
  (fp_line (start 5.05 -1.7) (end 5.05 -2.45) (stroke (width 0.12) (type solid)) (layer "F.SilkS"))
  (fp_line (start 3.25 -1.7) (end 5.05 -1.7) (stroke (width 0.12) (type solid)) (layer "F.SilkS"))
  (fp_line (start 1.75 -1.7) (end 1.75 -2.45) (stroke (width 0.12) (type solid)) (layer "F.SilkS"))
  (fp_line (start 0.75 -1.7) (end 1.75 -1.7) (stroke (width 0.12) (type solid)) (layer "F.SilkS"))
  (fp_line (start -0.75 -1.7) (end -0.75 -2.45) (stroke (width 0.12) (type solid)) (layer "F.SilkS"))
  (fp_line (start -2.55 -1.7) (end -0.75 -1.7) (stroke (width 0.12) (type solid)) (layer "F.SilkS"))
  (fp_line (start 5.05 -0.2) (end 4.3 -0.2) (stroke (width 0.12) (type solid)) (layer "F.SilkS"))
  (fp_line (start 4.3 -0.2) (end 4.3 2.75) (stroke (width 0.12) (type solid)) (layer "F.SilkS"))
  (fp_line (start -1.8 -0.2) (end -1.8 1.14) (stroke (width 0.12) (type solid)) (layer "F.SilkS"))
  (fp_line (start -2.55 -0.2) (end -1.8 -0.2) (stroke (width 0.12) (type solid)) (layer "F.SilkS"))
  (fp_line (start 4.3 2.75) (end 1.25 2.75) (stroke (width 0.12) (type solid)) (layer "F.SilkS"))
  (fp_line (start 1.25 2.75) (end -0.74 2.75) (stroke (width 0.12) (type solid)) (layer "F.SilkS"))
  (fp_line (start 5.06 3.51) (end 5.06 -2.46) (stroke (width 0.12) (type solid)) (layer "F.SilkS"))
  (fp_line (start -2.56 3.51) (end 5.06 3.51) (stroke (width 0.12) (type solid)) (layer "F.SilkS"))
  (pad "" np_thru_hole circle (at -1.6 2 90) (size 1.2 1.2) (drill 1.2) (layers "*.Cu" "*.Mask"))
  (pad "1" thru_hole roundrect (at 0 0 90) (size 1.7 2) (drill 1) (layers "*.Cu" "*.Mask") (remove_unused_layers no)
   (roundrect_rratio 0.147059) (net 51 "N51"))
  (pad "2" thru_hole oval (at 2.5 0 90) (size 1.7 2) (drill 1) (layers "*.Cu" "*.Mask") (remove_unused_layers no) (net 50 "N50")))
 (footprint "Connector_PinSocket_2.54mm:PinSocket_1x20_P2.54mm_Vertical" (layer "F.Cu") (at 149.5 118.2225 180)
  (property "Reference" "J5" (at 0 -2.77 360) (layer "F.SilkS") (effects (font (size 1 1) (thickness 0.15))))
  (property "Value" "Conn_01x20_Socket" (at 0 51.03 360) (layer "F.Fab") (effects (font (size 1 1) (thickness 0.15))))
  (fp_line (start 1.33 1.27) (end 1.33 49.59) (stroke (width 0.12) (type solid)) (layer "F.SilkS"))
  (fp_line (start 1.33 -1.33) (end 1.33 0) (stroke (width 0.12) (type solid)) (layer "F.SilkS"))
  (fp_line (start 0 -1.33) (end 1.33 -1.33) (stroke (width 0.12) (type solid)) (layer "F.SilkS"))
  (fp_line (start -1.33 49.59) (end 1.33 49.59) (stroke (width 0.12) (type solid)) (layer "F.SilkS"))
  (fp_line (start -1.33 1.27) (end 1.33 1.27) (stroke (width 0.12) (type solid)) (layer "F.SilkS"))
  (fp_line (start -1.33 1.27) (end -1.33 49.59) (stroke (width 0.12) (type solid)) (layer "F.SilkS"))
  (pad "1" thru_hole rect (at 0 0 180) (size 1.7 1.7) (drill 1) (layers "*.Cu" "*.Mask") (remove_unused_layers no) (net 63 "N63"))
  (pad "2" thru_hole oval (at 0 2.54 180) (size 1.7 1.7) (drill 1) (layers "*.Cu" "*.Mask") (remove_unused_layers no) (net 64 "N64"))
  (pad "3" thru_hole oval (at 0 5.08 180) (size 1.7 1.7) (drill 1) (layers "*.Cu" "*.Mask") (remove_unused_layers no) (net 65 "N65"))
  (pad "4" thru_hole oval (at 0 7.62 180) (size 1.7 1.7) (drill 1) (layers "*.Cu" "*.Mask") (remove_unused_layers no) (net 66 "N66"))
  (pad "5" thru_hole oval (at 0 10.16 180) (size 1.7 1.7) (drill 1) (layers "*.Cu" "*.Mask") (remove_unused_layers no) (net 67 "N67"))
  (pad "6" thru_hole oval (at 0 12.7 180) (size 1.7 1.7) (drill 1) (layers "*.Cu" "*.Mask") (remove_unused_layers no) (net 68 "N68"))
  (pad "7" thru_hole oval (at 0 15.24 180) (size 1.7 1.7) (drill 1) (layers "*.Cu" "*.Mask") (remove_unused_layers no) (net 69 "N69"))
  (pad "8" thru_hole oval (at 0 17.78 180) (size 1.7 1.7) (drill 1) (layers "*.Cu" "*.Mask") (remove_unused_layers no) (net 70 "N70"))
  (pad "9" thru_hole oval (at 0 20.32 180) (size 1.7 1.7) (drill 1) (layers "*.Cu" "*.Mask") (remove_unused_layers no) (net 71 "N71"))
  (pad "10" thru_hole oval (at 0 22.86 180) (size 1.7 1.7) (drill 1) (layers "*.Cu" "*.Mask") (remove_unused_layers no) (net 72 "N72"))
  (pad "11" thru_hole oval (at 0 25.4 180) (size 1.7 1.7) (drill 1) (layers "*.Cu" "*.Mask") (remove_unused_layers no) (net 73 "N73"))
  (pad "12" thru_hole oval (at 0 27.94 180) (size 1.7 1.7) (drill 1) (layers "*.Cu" "*.Mask") (remove_unused_layers no) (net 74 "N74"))
  (pad "13" thru_hole oval (at 0 30.48 180) (size 1.7 1.7) (drill 1) (layers "*.Cu" "*.Mask") (remove_unused_layers no) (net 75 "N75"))
  (pad "14" thru_hole oval (at 0 33.02 180) (size 1.7 1.7) (drill 1) (layers "*.Cu" "*.Mask") (remove_unused_layers no) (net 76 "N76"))
  (pad "15" thru_hole oval (at 0 35.56 180) (size 1.7 1.7) (drill 1) (layers "*.Cu" "*.Mask") (remove_unused_layers no) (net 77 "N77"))
  (pad "16" thru_hole oval (at 0 38.1 180) (size 1.7 1.7) (drill 1) (layers "*.Cu" "*.Mask") (remove_unused_layers no) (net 41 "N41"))
  (pad "17" thru_hole oval (at 0 40.64 180) (size 1.7 1.7) (drill 1) (layers "*.Cu" "*.Mask") (remove_unused_layers no) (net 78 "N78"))
  (pad "18" thru_hole oval (at 0 43.18 180) (size 1.7 1.7) (drill 1) (layers "*.Cu" "*.Mask") (remove_unused_layers no) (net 47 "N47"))
  (pad "19" thru_hole oval (at 0 45.72 180) (size 1.7 1.7) (drill 1) (layers "*.Cu" "*.Mask") (remove_unused_layers no) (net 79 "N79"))
  (pad "20" thru_hole oval (at 0 48.26 180) (size 1.7 1.7) (drill 1) (layers "*.Cu" "*.Mask") (remove_unused_layers no) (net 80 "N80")))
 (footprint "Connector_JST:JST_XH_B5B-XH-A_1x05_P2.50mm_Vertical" (layer "F.Cu") (at 167.64 101.76 -90)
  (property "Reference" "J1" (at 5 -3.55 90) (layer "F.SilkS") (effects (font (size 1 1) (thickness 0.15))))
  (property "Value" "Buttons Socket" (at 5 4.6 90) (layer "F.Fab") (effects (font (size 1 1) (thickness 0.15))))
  (fp_line (start -2.56 3.51) (end 12.56 3.51) (stroke (width 0.12) (type solid)) (layer "F.SilkS"))
  (fp_line (start 12.56 3.51) (end 12.56 -2.46) (stroke (width 0.12) (type solid)) (layer "F.SilkS"))
  (fp_line (start -1.8 2.75) (end 5 2.75) (stroke (width 0.12) (type solid)) (layer "F.SilkS"))
  (fp_line (start 11.8 2.75) (end 5 2.75) (stroke (width 0.12) (type solid)) (layer "F.SilkS"))
  (fp_line (start -2.55 -0.2) (end -1.8 -0.2) (stroke (width 0.12) (type solid)) (layer "F.SilkS"))
  (fp_line (start -1.8 -0.2) (end -1.8 2.75) (stroke (width 0.12) (type solid)) (layer "F.SilkS"))
  (fp_line (start 11.8 -0.2) (end 11.8 2.75) (stroke (width 0.12) (type solid)) (layer "F.SilkS"))
  (fp_line (start 12.55 -0.2) (end 11.8 -0.2) (stroke (width 0.12) (type solid)) (layer "F.SilkS"))
  (fp_line (start -2.55 -1.7) (end -0.75 -1.7) (stroke (width 0.12) (type solid)) (layer "F.SilkS"))
  (fp_line (start -0.75 -1.7) (end -0.75 -2.45) (stroke (width 0.12) (type solid)) (layer "F.SilkS"))
  (fp_line (start 0.75 -1.7) (end 9.25 -1.7) (stroke (width 0.12) (type solid)) (layer "F.SilkS"))
  (fp_line (start 9.25 -1.7) (end 9.25 -2.45) (stroke (width 0.12) (type solid)) (layer "F.SilkS"))
  (fp_line (start 10.75 -1.7) (end 12.55 -1.7) (stroke (width 0.12) (type solid)) (layer "F.SilkS"))
  (fp_line (start 12.55 -1.7) (end 12.55 -2.45) (stroke (width 0.12) (type solid)) (layer "F.SilkS"))
  (fp_line (start -2.55 -2.45) (end -2.55 -1.7) (stroke (width 0.12) (type solid)) (layer "F.SilkS"))
  (fp_line (start -0.75 -2.45) (end -2.55 -2.45) (stroke (width 0.12) (type solid)) (layer "F.SilkS"))
  (fp_line (start 0.75 -2.45) (end 0.75 -1.7) (stroke (width 0.12) (type solid)) (layer "F.SilkS"))
  (fp_line (start 9.25 -2.45) (end 0.75 -2.45) (stroke (width 0.12) (type solid)) (layer "F.SilkS"))
  (fp_line (start 10.75 -2.45) (end 10.75 -1.7) (stroke (width 0.12) (type solid)) (layer "F.SilkS"))
  (fp_line (start 12.55 -2.45) (end 10.75 -2.45) (stroke (width 0.12) (type solid)) (layer "F.SilkS"))
  (fp_line (start -2.56 -2.46) (end -2.56 3.51) (stroke (width 0.12) (type solid)) (layer "F.SilkS"))
  (fp_line (start 12.56 -2.46) (end -2.56 -2.46) (stroke (width 0.12) (type solid)) (layer "F.SilkS"))
  (fp_line (start -2.85 -2.75) (end -2.85 -1.5) (stroke (width 0.12) (type solid)) (layer "F.SilkS"))
  (fp_line (start -1.6 -2.75) (end -2.85 -2.75) (stroke (width 0.12) (type solid)) (layer "F.SilkS"))
  (pad "1" thru_hole roundrect (at 0 0 270) (size 1.7 1.95) (drill 0.95) (layers "*.Cu" "*.Mask") (remove_unused_layers no)
   (roundrect_rratio 0.147059) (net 69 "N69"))
  (pad "2" thru_hole oval (at 2.5 0 270) (size 1.7 1.95) (drill 0.95) (layers "*.Cu" "*.Mask") (remove_unused_layers no) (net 68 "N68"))
  (pad "3" thru_hole oval (at 5 0 270) (size 1.7 1.95) (drill 0.95) (layers "*.Cu" "*.Mask") (remove_unused_layers no) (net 67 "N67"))
  (pad "4" thru_hole oval (at 7.5 0 270) (size 1.7 1.95) (drill 0.95) (layers "*.Cu" "*.Mask") (remove_unused_layers no) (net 66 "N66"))
  (pad "5" thru_hole oval (at 10 0 270) (size 1.7 1.95) (drill 0.95) (layers "*.Cu" "*.Mask") (remove_unused_layers no) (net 65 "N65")))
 (gr_rect (start 112.72 64.14) (end 172.72 144.14) (stroke (width 0.05) (type default)) (fill none) (layer "Edge.Cuts"))
 (segment (start 165.64 77.14) (end 164.0475 78.7325) (width 0.2) (layer "F.Cu") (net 51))
 (segment (start 164.0475 78.7325) (end 133.93 78.7325) (width 0.2) (layer "F.Cu") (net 51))
 (segment (start 133.93 78.7325) (end 132.82 77.6225) (width 0.2) (layer "F.Cu") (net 51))
 (segment (start 165.64 74.64) (end 164.0875 76.1925) (width 0.2) (layer "F.Cu") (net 50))
 (segment (start 133.940031 76.1925) (end 132.830031 75.0825) (width 0.2) (layer "F.Cu") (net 50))
 (segment (start 164.0875 76.1925) (end 133.940031 76.1925) (width 0.2) (layer "F.Cu") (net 50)))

